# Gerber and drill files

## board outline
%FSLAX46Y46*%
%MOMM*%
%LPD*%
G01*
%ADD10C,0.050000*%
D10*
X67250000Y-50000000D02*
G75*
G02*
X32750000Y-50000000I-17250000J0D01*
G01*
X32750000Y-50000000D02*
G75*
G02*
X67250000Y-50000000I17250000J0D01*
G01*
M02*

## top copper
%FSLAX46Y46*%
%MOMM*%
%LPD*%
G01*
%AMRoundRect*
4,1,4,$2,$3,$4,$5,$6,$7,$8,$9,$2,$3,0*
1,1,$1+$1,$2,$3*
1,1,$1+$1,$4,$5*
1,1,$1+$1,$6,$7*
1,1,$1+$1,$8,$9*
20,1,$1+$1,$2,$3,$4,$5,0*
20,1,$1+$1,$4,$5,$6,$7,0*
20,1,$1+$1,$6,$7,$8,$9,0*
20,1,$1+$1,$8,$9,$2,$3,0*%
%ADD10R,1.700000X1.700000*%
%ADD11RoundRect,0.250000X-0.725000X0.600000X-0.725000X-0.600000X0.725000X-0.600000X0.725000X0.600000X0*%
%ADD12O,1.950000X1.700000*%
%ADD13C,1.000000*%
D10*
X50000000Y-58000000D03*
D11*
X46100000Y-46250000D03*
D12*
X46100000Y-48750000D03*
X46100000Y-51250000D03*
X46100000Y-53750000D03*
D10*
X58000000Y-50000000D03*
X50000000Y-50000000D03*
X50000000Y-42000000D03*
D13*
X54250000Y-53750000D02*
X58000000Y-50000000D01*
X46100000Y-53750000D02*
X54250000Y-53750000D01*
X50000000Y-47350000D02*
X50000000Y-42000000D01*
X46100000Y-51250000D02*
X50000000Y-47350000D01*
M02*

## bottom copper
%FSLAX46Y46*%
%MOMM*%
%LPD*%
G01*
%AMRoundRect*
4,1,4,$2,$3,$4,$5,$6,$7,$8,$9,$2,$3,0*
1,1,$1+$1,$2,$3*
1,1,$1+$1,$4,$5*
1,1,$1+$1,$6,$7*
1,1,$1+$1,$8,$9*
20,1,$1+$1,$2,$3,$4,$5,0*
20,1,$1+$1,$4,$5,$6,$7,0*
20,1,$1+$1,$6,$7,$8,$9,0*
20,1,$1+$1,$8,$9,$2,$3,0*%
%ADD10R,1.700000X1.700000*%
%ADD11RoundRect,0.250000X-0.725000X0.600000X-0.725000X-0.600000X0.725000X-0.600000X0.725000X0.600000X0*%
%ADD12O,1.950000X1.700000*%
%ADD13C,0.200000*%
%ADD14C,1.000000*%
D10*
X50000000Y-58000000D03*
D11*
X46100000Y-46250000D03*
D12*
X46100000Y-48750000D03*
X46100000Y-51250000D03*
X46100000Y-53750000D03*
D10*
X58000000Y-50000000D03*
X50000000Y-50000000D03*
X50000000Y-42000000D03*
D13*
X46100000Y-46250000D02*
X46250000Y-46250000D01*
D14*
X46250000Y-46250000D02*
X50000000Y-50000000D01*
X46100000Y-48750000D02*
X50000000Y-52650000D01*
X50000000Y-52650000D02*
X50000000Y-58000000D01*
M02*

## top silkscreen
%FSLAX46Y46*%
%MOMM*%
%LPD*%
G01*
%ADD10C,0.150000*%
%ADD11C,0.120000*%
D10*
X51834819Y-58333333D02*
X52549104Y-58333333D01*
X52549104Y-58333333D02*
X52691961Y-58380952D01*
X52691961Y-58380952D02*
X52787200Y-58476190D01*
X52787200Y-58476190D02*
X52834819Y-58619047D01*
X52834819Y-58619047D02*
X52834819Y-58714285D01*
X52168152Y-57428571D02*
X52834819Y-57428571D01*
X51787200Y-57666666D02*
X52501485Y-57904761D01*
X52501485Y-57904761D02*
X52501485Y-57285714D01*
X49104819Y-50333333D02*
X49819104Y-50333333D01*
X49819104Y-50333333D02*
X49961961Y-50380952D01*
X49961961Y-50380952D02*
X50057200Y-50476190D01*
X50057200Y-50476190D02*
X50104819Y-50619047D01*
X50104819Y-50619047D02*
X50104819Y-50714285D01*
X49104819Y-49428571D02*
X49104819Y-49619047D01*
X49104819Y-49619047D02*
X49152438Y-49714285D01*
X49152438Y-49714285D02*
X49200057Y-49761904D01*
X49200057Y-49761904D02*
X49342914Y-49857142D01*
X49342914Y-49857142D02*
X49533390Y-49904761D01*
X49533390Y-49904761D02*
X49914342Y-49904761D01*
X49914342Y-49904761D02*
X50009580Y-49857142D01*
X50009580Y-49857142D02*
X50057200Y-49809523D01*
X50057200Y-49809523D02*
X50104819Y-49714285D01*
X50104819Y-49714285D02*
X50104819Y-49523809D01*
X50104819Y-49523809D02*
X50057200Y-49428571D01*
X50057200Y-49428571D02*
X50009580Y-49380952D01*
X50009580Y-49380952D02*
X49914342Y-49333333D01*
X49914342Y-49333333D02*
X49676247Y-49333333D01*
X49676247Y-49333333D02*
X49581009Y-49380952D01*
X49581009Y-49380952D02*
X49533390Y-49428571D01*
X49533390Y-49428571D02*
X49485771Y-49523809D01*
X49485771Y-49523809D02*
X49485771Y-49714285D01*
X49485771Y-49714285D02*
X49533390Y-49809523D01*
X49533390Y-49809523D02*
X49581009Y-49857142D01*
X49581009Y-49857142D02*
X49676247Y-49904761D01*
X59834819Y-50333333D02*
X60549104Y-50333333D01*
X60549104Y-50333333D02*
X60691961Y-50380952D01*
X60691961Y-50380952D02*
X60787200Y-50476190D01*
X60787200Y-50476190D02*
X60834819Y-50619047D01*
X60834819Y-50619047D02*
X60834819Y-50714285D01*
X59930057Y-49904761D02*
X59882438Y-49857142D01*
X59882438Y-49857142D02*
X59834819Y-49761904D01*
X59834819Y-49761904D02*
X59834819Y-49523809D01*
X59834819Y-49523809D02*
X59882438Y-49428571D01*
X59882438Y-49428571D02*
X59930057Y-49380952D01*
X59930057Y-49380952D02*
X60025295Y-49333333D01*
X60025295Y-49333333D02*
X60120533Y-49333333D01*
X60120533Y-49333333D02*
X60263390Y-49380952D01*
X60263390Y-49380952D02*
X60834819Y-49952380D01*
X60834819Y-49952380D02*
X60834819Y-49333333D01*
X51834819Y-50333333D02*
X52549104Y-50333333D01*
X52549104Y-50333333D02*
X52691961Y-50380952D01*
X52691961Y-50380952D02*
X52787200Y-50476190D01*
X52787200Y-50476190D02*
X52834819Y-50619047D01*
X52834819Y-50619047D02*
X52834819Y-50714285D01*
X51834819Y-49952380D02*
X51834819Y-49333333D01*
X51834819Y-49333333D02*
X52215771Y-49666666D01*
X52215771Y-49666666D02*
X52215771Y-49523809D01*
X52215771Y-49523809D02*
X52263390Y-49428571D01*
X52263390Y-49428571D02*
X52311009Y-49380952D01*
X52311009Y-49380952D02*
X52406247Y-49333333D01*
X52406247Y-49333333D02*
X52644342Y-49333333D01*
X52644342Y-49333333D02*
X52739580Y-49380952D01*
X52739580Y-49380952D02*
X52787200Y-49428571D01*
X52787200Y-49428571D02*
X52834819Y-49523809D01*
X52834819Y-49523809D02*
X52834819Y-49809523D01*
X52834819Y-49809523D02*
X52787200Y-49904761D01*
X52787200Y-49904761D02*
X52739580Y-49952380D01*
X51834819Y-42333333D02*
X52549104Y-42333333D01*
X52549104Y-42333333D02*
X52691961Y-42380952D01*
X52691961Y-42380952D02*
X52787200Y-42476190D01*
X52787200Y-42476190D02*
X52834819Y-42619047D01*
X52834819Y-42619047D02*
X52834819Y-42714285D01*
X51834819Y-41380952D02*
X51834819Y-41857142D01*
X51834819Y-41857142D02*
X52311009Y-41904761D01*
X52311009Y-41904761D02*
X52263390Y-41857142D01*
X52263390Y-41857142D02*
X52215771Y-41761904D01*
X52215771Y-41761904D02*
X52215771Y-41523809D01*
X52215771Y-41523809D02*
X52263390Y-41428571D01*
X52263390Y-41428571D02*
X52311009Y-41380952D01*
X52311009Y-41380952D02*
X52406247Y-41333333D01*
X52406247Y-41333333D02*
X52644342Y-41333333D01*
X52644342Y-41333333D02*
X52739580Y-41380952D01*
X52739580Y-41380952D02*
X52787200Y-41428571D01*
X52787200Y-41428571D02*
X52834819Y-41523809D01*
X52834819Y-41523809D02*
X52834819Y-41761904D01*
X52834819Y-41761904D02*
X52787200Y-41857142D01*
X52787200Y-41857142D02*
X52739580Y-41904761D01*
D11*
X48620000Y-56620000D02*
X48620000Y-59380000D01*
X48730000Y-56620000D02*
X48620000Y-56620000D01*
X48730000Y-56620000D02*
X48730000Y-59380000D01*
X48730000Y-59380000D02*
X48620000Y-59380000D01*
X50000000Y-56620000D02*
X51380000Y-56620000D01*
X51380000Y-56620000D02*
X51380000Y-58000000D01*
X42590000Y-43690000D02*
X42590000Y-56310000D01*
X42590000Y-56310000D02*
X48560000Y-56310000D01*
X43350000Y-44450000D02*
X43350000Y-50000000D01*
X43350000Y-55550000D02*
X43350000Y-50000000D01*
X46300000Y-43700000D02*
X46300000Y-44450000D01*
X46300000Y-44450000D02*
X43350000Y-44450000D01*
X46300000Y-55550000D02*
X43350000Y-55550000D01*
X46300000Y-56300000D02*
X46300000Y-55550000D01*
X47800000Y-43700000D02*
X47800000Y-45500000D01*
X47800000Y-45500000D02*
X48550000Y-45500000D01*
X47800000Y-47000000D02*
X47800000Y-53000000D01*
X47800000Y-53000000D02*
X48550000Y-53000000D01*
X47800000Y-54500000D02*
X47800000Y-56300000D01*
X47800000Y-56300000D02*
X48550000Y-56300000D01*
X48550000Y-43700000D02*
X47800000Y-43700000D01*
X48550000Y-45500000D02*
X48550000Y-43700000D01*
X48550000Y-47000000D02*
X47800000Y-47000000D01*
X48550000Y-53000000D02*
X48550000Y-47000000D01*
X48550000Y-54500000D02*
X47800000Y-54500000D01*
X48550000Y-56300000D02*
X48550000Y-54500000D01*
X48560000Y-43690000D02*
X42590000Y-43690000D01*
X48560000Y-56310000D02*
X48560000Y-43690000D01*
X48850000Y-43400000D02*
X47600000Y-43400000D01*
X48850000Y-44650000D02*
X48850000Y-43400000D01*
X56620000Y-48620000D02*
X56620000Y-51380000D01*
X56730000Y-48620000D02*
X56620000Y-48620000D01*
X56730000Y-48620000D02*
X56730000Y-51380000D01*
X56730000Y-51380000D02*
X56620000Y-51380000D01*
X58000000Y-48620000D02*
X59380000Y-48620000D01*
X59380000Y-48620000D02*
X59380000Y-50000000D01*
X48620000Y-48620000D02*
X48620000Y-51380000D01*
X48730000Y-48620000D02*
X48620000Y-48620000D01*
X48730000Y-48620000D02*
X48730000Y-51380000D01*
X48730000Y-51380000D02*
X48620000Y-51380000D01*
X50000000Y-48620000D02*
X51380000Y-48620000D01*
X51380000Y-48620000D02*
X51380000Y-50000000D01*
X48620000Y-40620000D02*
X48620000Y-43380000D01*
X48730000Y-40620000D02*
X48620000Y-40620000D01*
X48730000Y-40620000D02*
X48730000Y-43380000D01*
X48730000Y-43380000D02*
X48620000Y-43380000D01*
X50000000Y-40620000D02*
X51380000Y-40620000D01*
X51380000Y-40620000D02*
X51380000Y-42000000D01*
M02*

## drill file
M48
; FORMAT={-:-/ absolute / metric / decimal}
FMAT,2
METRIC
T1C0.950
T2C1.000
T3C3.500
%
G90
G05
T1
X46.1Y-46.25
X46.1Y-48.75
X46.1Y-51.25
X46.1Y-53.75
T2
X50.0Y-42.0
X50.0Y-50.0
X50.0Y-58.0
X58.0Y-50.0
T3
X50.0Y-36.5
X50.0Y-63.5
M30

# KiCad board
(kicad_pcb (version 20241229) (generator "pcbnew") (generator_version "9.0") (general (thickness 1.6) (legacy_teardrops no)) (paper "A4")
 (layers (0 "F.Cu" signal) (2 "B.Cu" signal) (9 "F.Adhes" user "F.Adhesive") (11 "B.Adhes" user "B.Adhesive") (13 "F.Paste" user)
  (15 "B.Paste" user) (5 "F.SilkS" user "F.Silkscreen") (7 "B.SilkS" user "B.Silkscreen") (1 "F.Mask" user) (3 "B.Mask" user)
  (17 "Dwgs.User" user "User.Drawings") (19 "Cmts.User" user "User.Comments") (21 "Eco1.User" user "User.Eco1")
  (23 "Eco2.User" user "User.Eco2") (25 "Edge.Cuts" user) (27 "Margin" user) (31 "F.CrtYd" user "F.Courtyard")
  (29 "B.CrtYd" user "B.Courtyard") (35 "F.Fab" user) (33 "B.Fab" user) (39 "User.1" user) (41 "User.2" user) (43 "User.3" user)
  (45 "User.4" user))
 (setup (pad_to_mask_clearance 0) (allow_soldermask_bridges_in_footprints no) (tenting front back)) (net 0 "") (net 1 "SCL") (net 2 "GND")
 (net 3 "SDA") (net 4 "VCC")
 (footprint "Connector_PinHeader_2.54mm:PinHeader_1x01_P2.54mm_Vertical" (layer "F.Cu") (at 50 58 -90)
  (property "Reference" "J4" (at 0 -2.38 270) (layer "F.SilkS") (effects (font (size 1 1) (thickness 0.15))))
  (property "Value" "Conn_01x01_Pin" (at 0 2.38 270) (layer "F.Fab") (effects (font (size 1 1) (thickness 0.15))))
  (fp_line (start -1.38 1.38) (end 1.38 1.38) (stroke (width 0.12) (type solid)) (layer "F.SilkS"))
  (fp_line (start -1.38 1.27) (end -1.38 1.38) (stroke (width 0.12) (type solid)) (layer "F.SilkS"))
  (fp_line (start -1.38 1.27) (end 1.38 1.27) (stroke (width 0.12) (type solid)) (layer "F.SilkS"))
  (fp_line (start 1.38 1.27) (end 1.38 1.38) (stroke (width 0.12) (type solid)) (layer "F.SilkS"))
  (fp_line (start -1.38 0) (end -1.38 -1.38) (stroke (width 0.12) (type solid)) (layer "F.SilkS"))
  (fp_line (start -1.38 -1.38) (end 0 -1.38) (stroke (width 0.12) (type solid)) (layer "F.SilkS"))
  (pad "1" thru_hole rect (at 0 0 270) (size 1.7 1.7) (drill 1) (layers "*.Cu" "*.Mask") (remove_unused_layers no) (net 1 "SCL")))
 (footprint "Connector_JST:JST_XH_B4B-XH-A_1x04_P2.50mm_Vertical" (layer "F.Cu") (at 46.1 46.25 -90)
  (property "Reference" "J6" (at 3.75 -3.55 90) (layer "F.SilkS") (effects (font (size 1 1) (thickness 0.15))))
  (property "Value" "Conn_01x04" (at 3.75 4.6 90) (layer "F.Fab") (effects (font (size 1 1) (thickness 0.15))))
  (fp_line (start -2.56 3.51) (end 10.06 3.51) (stroke (width 0.12) (type solid)) (layer "F.SilkS"))
  (fp_line (start 10.06 3.51) (end 10.06 -2.46) (stroke (width 0.12) (type solid)) (layer "F.SilkS"))
  (fp_line (start -1.8 2.75) (end 3.75 2.75) (stroke (width 0.12) (type solid)) (layer "F.SilkS"))
  (fp_line (start 9.3 2.75) (end 3.75 2.75) (stroke (width 0.12) (type solid)) (layer "F.SilkS"))
  (fp_line (start -2.55 -0.2) (end -1.8 -0.2) (stroke (width 0.12) (type solid)) (layer "F.SilkS"))
  (fp_line (start -1.8 -0.2) (end -1.8 2.75) (stroke (width 0.12) (type solid)) (layer "F.SilkS"))
  (fp_line (start 9.3 -0.2) (end 9.3 2.75) (stroke (width 0.12) (type solid)) (layer "F.SilkS"))
  (fp_line (start 10.05 -0.2) (end 9.3 -0.2) (stroke (width 0.12) (type solid)) (layer "F.SilkS"))
  (fp_line (start -2.55 -1.7) (end -0.75 -1.7) (stroke (width 0.12) (type solid)) (layer "F.SilkS"))
  (fp_line (start -0.75 -1.7) (end -0.75 -2.45) (stroke (width 0.12) (type solid)) (layer "F.SilkS"))
  (fp_line (start 0.75 -1.7) (end 6.75 -1.7) (stroke (width 0.12) (type solid)) (layer "F.SilkS"))
  (fp_line (start 6.75 -1.7) (end 6.75 -2.45) (stroke (width 0.12) (type solid)) (layer "F.SilkS"))
  (fp_line (start 8.25 -1.7) (end 10.05 -1.7) (stroke (width 0.12) (type solid)) (layer "F.SilkS"))
  (fp_line (start 10.05 -1.7) (end 10.05 -2.45) (stroke (width 0.12) (type solid)) (layer "F.SilkS"))
  (fp_line (start -2.55 -2.45) (end -2.55 -1.7) (stroke (width 0.12) (type solid)) (layer "F.SilkS"))
  (fp_line (start -0.75 -2.45) (end -2.55 -2.45) (stroke (width 0.12) (type solid)) (layer "F.SilkS"))
  (fp_line (start 0.75 -2.45) (end 0.75 -1.7) (stroke (width 0.12) (type solid)) (layer "F.SilkS"))
  (fp_line (start 6.75 -2.45) (end 0.75 -2.45) (stroke (width 0.12) (type solid)) (layer "F.SilkS"))
  (fp_line (start 8.25 -2.45) (end 8.25 -1.7) (stroke (width 0.12) (type solid)) (layer "F.SilkS"))
  (fp_line (start 10.05 -2.45) (end 8.25 -2.45) (stroke (width 0.12) (type solid)) (layer "F.SilkS"))
  (fp_line (start -2.56 -2.46) (end -2.56 3.51) (stroke (width 0.12) (type solid)) (layer "F.SilkS"))
  (fp_line (start 10.06 -2.46) (end -2.56 -2.46) (stroke (width 0.12) (type solid)) (layer "F.SilkS"))
  (fp_line (start -2.85 -2.75) (end -2.85 -1.5) (stroke (width 0.12) (type solid)) (layer "F.SilkS"))
  (fp_line (start -1.6 -2.75) (end -2.85 -2.75) (stroke (width 0.12) (type solid)) (layer "F.SilkS"))
  (pad "1" thru_hole roundrect (at 0 0 270) (size 1.7 1.95) (drill 0.95) (layers "*.Cu" "*.Mask") (remove_unused_layers no)
   (roundrect_rratio 0.147059) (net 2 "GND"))
  (pad "2" thru_hole oval (at 2.5 0 270) (size 1.7 1.95) (drill 0.95) (layers "*.Cu" "*.Mask") (remove_unused_layers no) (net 1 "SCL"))
  (pad "3" thru_hole oval (at 5 0 270) (size 1.7 1.95) (drill 0.95) (layers "*.Cu" "*.Mask") (remove_unused_layers no) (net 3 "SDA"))
  (pad "4" thru_hole oval (at 7.5 0 270) (size 1.7 1.95) (drill 0.95) (layers "*.Cu" "*.Mask") (remove_unused_layers no) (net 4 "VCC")))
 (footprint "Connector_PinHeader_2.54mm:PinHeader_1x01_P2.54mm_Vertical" (layer "F.Cu") (at 58 50 -90)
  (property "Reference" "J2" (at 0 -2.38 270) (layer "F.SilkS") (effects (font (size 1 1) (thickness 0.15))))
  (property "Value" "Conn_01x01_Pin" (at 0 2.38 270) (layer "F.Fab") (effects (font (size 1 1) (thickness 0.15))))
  (fp_line (start -1.38 1.38) (end 1.38 1.38) (stroke (width 0.12) (type solid)) (layer "F.SilkS"))
  (fp_line (start -1.38 1.27) (end -1.38 1.38) (stroke (width 0.12) (type solid)) (layer "F.SilkS"))
  (fp_line (start -1.38 1.27) (end 1.38 1.27) (stroke (width 0.12) (type solid)) (layer "F.SilkS"))
  (fp_line (start 1.38 1.27) (end 1.38 1.38) (stroke (width 0.12) (type solid)) (layer "F.SilkS"))
  (fp_line (start -1.38 0) (end -1.38 -1.38) (stroke (width 0.12) (type solid)) (layer "F.SilkS"))
  (fp_line (start -1.38 -1.38) (end 0 -1.38) (stroke (width 0.12) (type solid)) (layer "F.SilkS"))
  (pad "1" thru_hole rect (at 0 0 270) (size 1.7 1.7) (drill 1) (layers "*.Cu" "*.Mask") (remove_unused_layers no) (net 4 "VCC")))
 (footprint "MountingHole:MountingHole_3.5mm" (layer "F.Cu") (at 50 36.5)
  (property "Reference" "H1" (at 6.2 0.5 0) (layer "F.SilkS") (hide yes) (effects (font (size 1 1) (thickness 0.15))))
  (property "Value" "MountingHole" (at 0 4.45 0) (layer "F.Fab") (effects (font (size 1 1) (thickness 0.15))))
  (pad "" np_thru_hole circle (at 0 0) (size 3.5 3.5) (drill 3.5) (layers "*.Cu" "*.Mask")))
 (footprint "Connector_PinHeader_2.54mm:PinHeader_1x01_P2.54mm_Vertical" (layer "F.Cu") (at 50 50 -90)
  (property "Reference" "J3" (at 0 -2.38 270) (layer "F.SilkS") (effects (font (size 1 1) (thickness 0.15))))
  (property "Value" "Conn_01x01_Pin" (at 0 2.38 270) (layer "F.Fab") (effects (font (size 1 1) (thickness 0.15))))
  (fp_line (start -1.38 1.38) (end 1.38 1.38) (stroke (width 0.12) (type solid)) (layer "F.SilkS"))
  (fp_line (start -1.38 1.27) (end -1.38 1.38) (stroke (width 0.12) (type solid)) (layer "F.SilkS"))
  (fp_line (start -1.38 1.27) (end 1.38 1.27) (stroke (width 0.12) (type solid)) (layer "F.SilkS"))
  (fp_line (start 1.38 1.27) (end 1.38 1.38) (stroke (width 0.12) (type solid)) (layer "F.SilkS"))
  (fp_line (start -1.38 0) (end -1.38 -1.38) (stroke (width 0.12) (type solid)) (layer "F.SilkS"))
  (fp_line (start -1.38 -1.38) (end 0 -1.38) (stroke (width 0.12) (type solid)) (layer "F.SilkS"))
  (pad "1" thru_hole rect (at 0 0 270) (size 1.7 1.7) (drill 1) (layers "*.Cu" "*.Mask") (remove_unused_layers no) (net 2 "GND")))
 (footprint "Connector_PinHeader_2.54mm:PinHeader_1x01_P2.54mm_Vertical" (layer "F.Cu") (at 50 42 -90)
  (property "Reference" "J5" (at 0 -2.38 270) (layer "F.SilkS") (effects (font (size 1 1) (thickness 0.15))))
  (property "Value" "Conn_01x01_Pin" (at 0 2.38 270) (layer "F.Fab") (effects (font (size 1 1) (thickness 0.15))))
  (fp_line (start -1.38 1.38) (end 1.38 1.38) (stroke (width 0.12) (type solid)) (layer "F.SilkS"))
  (fp_line (start -1.38 1.27) (end -1.38 1.38) (stroke (width 0.12) (type solid)) (layer "F.SilkS"))
  (fp_line (start -1.38 1.27) (end 1.38 1.27) (stroke (width 0.12) (type solid)) (layer "F.SilkS"))
  (fp_line (start 1.38 1.27) (end 1.38 1.38) (stroke (width 0.12) (type solid)) (layer "F.SilkS"))
  (fp_line (start -1.38 0) (end -1.38 -1.38) (stroke (width 0.12) (type solid)) (layer "F.SilkS"))
  (fp_line (start -1.38 -1.38) (end 0 -1.38) (stroke (width 0.12) (type solid)) (layer "F.SilkS"))
  (pad "1" thru_hole rect (at 0 0 270) (size 1.7 1.7) (drill 1) (layers "*.Cu" "*.Mask") (remove_unused_layers no) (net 3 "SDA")))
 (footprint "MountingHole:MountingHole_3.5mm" (layer "F.Cu") (at 50 63.5)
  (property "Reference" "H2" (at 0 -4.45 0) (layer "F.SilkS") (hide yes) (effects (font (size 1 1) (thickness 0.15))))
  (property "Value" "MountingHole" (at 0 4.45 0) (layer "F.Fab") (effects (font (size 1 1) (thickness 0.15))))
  (pad "" np_thru_hole circle (at 0 0) (size 3.5 3.5) (drill 3.5) (layers "*.Cu" "*.Mask")))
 (gr_circle (center 50 50) (end 67.25 50) (stroke (width 0.05) (type solid)) (fill no) (layer "Edge.Cuts"))
 (segment (start 54.25 53.75) (end 58 50) (width 1) (layer "F.Cu") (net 4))
 (segment (start 46.1 53.75) (end 54.25 53.75) (width 1) (layer "F.Cu") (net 4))
 (segment (start 46.1 46.25) (end 46.25 46.25) (width 0.2) (layer "B.Cu") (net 2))
 (segment (start 46.25 46.25) (end 50 50) (width 1) (layer "B.Cu") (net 2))
 (segment (start 46.1 48.75) (end 50 52.65) (width 1) (layer "B.Cu") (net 1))
 (segment (start 50 52.65) (end 50 58) (width 1) (layer "B.Cu") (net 1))
 (segment (start 50 47.35) (end 50 42) (width 1) (layer "F.Cu") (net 3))
 (segment (start 46.1 51.25) (end 50 47.35) (width 1) (layer "F.Cu") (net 3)))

